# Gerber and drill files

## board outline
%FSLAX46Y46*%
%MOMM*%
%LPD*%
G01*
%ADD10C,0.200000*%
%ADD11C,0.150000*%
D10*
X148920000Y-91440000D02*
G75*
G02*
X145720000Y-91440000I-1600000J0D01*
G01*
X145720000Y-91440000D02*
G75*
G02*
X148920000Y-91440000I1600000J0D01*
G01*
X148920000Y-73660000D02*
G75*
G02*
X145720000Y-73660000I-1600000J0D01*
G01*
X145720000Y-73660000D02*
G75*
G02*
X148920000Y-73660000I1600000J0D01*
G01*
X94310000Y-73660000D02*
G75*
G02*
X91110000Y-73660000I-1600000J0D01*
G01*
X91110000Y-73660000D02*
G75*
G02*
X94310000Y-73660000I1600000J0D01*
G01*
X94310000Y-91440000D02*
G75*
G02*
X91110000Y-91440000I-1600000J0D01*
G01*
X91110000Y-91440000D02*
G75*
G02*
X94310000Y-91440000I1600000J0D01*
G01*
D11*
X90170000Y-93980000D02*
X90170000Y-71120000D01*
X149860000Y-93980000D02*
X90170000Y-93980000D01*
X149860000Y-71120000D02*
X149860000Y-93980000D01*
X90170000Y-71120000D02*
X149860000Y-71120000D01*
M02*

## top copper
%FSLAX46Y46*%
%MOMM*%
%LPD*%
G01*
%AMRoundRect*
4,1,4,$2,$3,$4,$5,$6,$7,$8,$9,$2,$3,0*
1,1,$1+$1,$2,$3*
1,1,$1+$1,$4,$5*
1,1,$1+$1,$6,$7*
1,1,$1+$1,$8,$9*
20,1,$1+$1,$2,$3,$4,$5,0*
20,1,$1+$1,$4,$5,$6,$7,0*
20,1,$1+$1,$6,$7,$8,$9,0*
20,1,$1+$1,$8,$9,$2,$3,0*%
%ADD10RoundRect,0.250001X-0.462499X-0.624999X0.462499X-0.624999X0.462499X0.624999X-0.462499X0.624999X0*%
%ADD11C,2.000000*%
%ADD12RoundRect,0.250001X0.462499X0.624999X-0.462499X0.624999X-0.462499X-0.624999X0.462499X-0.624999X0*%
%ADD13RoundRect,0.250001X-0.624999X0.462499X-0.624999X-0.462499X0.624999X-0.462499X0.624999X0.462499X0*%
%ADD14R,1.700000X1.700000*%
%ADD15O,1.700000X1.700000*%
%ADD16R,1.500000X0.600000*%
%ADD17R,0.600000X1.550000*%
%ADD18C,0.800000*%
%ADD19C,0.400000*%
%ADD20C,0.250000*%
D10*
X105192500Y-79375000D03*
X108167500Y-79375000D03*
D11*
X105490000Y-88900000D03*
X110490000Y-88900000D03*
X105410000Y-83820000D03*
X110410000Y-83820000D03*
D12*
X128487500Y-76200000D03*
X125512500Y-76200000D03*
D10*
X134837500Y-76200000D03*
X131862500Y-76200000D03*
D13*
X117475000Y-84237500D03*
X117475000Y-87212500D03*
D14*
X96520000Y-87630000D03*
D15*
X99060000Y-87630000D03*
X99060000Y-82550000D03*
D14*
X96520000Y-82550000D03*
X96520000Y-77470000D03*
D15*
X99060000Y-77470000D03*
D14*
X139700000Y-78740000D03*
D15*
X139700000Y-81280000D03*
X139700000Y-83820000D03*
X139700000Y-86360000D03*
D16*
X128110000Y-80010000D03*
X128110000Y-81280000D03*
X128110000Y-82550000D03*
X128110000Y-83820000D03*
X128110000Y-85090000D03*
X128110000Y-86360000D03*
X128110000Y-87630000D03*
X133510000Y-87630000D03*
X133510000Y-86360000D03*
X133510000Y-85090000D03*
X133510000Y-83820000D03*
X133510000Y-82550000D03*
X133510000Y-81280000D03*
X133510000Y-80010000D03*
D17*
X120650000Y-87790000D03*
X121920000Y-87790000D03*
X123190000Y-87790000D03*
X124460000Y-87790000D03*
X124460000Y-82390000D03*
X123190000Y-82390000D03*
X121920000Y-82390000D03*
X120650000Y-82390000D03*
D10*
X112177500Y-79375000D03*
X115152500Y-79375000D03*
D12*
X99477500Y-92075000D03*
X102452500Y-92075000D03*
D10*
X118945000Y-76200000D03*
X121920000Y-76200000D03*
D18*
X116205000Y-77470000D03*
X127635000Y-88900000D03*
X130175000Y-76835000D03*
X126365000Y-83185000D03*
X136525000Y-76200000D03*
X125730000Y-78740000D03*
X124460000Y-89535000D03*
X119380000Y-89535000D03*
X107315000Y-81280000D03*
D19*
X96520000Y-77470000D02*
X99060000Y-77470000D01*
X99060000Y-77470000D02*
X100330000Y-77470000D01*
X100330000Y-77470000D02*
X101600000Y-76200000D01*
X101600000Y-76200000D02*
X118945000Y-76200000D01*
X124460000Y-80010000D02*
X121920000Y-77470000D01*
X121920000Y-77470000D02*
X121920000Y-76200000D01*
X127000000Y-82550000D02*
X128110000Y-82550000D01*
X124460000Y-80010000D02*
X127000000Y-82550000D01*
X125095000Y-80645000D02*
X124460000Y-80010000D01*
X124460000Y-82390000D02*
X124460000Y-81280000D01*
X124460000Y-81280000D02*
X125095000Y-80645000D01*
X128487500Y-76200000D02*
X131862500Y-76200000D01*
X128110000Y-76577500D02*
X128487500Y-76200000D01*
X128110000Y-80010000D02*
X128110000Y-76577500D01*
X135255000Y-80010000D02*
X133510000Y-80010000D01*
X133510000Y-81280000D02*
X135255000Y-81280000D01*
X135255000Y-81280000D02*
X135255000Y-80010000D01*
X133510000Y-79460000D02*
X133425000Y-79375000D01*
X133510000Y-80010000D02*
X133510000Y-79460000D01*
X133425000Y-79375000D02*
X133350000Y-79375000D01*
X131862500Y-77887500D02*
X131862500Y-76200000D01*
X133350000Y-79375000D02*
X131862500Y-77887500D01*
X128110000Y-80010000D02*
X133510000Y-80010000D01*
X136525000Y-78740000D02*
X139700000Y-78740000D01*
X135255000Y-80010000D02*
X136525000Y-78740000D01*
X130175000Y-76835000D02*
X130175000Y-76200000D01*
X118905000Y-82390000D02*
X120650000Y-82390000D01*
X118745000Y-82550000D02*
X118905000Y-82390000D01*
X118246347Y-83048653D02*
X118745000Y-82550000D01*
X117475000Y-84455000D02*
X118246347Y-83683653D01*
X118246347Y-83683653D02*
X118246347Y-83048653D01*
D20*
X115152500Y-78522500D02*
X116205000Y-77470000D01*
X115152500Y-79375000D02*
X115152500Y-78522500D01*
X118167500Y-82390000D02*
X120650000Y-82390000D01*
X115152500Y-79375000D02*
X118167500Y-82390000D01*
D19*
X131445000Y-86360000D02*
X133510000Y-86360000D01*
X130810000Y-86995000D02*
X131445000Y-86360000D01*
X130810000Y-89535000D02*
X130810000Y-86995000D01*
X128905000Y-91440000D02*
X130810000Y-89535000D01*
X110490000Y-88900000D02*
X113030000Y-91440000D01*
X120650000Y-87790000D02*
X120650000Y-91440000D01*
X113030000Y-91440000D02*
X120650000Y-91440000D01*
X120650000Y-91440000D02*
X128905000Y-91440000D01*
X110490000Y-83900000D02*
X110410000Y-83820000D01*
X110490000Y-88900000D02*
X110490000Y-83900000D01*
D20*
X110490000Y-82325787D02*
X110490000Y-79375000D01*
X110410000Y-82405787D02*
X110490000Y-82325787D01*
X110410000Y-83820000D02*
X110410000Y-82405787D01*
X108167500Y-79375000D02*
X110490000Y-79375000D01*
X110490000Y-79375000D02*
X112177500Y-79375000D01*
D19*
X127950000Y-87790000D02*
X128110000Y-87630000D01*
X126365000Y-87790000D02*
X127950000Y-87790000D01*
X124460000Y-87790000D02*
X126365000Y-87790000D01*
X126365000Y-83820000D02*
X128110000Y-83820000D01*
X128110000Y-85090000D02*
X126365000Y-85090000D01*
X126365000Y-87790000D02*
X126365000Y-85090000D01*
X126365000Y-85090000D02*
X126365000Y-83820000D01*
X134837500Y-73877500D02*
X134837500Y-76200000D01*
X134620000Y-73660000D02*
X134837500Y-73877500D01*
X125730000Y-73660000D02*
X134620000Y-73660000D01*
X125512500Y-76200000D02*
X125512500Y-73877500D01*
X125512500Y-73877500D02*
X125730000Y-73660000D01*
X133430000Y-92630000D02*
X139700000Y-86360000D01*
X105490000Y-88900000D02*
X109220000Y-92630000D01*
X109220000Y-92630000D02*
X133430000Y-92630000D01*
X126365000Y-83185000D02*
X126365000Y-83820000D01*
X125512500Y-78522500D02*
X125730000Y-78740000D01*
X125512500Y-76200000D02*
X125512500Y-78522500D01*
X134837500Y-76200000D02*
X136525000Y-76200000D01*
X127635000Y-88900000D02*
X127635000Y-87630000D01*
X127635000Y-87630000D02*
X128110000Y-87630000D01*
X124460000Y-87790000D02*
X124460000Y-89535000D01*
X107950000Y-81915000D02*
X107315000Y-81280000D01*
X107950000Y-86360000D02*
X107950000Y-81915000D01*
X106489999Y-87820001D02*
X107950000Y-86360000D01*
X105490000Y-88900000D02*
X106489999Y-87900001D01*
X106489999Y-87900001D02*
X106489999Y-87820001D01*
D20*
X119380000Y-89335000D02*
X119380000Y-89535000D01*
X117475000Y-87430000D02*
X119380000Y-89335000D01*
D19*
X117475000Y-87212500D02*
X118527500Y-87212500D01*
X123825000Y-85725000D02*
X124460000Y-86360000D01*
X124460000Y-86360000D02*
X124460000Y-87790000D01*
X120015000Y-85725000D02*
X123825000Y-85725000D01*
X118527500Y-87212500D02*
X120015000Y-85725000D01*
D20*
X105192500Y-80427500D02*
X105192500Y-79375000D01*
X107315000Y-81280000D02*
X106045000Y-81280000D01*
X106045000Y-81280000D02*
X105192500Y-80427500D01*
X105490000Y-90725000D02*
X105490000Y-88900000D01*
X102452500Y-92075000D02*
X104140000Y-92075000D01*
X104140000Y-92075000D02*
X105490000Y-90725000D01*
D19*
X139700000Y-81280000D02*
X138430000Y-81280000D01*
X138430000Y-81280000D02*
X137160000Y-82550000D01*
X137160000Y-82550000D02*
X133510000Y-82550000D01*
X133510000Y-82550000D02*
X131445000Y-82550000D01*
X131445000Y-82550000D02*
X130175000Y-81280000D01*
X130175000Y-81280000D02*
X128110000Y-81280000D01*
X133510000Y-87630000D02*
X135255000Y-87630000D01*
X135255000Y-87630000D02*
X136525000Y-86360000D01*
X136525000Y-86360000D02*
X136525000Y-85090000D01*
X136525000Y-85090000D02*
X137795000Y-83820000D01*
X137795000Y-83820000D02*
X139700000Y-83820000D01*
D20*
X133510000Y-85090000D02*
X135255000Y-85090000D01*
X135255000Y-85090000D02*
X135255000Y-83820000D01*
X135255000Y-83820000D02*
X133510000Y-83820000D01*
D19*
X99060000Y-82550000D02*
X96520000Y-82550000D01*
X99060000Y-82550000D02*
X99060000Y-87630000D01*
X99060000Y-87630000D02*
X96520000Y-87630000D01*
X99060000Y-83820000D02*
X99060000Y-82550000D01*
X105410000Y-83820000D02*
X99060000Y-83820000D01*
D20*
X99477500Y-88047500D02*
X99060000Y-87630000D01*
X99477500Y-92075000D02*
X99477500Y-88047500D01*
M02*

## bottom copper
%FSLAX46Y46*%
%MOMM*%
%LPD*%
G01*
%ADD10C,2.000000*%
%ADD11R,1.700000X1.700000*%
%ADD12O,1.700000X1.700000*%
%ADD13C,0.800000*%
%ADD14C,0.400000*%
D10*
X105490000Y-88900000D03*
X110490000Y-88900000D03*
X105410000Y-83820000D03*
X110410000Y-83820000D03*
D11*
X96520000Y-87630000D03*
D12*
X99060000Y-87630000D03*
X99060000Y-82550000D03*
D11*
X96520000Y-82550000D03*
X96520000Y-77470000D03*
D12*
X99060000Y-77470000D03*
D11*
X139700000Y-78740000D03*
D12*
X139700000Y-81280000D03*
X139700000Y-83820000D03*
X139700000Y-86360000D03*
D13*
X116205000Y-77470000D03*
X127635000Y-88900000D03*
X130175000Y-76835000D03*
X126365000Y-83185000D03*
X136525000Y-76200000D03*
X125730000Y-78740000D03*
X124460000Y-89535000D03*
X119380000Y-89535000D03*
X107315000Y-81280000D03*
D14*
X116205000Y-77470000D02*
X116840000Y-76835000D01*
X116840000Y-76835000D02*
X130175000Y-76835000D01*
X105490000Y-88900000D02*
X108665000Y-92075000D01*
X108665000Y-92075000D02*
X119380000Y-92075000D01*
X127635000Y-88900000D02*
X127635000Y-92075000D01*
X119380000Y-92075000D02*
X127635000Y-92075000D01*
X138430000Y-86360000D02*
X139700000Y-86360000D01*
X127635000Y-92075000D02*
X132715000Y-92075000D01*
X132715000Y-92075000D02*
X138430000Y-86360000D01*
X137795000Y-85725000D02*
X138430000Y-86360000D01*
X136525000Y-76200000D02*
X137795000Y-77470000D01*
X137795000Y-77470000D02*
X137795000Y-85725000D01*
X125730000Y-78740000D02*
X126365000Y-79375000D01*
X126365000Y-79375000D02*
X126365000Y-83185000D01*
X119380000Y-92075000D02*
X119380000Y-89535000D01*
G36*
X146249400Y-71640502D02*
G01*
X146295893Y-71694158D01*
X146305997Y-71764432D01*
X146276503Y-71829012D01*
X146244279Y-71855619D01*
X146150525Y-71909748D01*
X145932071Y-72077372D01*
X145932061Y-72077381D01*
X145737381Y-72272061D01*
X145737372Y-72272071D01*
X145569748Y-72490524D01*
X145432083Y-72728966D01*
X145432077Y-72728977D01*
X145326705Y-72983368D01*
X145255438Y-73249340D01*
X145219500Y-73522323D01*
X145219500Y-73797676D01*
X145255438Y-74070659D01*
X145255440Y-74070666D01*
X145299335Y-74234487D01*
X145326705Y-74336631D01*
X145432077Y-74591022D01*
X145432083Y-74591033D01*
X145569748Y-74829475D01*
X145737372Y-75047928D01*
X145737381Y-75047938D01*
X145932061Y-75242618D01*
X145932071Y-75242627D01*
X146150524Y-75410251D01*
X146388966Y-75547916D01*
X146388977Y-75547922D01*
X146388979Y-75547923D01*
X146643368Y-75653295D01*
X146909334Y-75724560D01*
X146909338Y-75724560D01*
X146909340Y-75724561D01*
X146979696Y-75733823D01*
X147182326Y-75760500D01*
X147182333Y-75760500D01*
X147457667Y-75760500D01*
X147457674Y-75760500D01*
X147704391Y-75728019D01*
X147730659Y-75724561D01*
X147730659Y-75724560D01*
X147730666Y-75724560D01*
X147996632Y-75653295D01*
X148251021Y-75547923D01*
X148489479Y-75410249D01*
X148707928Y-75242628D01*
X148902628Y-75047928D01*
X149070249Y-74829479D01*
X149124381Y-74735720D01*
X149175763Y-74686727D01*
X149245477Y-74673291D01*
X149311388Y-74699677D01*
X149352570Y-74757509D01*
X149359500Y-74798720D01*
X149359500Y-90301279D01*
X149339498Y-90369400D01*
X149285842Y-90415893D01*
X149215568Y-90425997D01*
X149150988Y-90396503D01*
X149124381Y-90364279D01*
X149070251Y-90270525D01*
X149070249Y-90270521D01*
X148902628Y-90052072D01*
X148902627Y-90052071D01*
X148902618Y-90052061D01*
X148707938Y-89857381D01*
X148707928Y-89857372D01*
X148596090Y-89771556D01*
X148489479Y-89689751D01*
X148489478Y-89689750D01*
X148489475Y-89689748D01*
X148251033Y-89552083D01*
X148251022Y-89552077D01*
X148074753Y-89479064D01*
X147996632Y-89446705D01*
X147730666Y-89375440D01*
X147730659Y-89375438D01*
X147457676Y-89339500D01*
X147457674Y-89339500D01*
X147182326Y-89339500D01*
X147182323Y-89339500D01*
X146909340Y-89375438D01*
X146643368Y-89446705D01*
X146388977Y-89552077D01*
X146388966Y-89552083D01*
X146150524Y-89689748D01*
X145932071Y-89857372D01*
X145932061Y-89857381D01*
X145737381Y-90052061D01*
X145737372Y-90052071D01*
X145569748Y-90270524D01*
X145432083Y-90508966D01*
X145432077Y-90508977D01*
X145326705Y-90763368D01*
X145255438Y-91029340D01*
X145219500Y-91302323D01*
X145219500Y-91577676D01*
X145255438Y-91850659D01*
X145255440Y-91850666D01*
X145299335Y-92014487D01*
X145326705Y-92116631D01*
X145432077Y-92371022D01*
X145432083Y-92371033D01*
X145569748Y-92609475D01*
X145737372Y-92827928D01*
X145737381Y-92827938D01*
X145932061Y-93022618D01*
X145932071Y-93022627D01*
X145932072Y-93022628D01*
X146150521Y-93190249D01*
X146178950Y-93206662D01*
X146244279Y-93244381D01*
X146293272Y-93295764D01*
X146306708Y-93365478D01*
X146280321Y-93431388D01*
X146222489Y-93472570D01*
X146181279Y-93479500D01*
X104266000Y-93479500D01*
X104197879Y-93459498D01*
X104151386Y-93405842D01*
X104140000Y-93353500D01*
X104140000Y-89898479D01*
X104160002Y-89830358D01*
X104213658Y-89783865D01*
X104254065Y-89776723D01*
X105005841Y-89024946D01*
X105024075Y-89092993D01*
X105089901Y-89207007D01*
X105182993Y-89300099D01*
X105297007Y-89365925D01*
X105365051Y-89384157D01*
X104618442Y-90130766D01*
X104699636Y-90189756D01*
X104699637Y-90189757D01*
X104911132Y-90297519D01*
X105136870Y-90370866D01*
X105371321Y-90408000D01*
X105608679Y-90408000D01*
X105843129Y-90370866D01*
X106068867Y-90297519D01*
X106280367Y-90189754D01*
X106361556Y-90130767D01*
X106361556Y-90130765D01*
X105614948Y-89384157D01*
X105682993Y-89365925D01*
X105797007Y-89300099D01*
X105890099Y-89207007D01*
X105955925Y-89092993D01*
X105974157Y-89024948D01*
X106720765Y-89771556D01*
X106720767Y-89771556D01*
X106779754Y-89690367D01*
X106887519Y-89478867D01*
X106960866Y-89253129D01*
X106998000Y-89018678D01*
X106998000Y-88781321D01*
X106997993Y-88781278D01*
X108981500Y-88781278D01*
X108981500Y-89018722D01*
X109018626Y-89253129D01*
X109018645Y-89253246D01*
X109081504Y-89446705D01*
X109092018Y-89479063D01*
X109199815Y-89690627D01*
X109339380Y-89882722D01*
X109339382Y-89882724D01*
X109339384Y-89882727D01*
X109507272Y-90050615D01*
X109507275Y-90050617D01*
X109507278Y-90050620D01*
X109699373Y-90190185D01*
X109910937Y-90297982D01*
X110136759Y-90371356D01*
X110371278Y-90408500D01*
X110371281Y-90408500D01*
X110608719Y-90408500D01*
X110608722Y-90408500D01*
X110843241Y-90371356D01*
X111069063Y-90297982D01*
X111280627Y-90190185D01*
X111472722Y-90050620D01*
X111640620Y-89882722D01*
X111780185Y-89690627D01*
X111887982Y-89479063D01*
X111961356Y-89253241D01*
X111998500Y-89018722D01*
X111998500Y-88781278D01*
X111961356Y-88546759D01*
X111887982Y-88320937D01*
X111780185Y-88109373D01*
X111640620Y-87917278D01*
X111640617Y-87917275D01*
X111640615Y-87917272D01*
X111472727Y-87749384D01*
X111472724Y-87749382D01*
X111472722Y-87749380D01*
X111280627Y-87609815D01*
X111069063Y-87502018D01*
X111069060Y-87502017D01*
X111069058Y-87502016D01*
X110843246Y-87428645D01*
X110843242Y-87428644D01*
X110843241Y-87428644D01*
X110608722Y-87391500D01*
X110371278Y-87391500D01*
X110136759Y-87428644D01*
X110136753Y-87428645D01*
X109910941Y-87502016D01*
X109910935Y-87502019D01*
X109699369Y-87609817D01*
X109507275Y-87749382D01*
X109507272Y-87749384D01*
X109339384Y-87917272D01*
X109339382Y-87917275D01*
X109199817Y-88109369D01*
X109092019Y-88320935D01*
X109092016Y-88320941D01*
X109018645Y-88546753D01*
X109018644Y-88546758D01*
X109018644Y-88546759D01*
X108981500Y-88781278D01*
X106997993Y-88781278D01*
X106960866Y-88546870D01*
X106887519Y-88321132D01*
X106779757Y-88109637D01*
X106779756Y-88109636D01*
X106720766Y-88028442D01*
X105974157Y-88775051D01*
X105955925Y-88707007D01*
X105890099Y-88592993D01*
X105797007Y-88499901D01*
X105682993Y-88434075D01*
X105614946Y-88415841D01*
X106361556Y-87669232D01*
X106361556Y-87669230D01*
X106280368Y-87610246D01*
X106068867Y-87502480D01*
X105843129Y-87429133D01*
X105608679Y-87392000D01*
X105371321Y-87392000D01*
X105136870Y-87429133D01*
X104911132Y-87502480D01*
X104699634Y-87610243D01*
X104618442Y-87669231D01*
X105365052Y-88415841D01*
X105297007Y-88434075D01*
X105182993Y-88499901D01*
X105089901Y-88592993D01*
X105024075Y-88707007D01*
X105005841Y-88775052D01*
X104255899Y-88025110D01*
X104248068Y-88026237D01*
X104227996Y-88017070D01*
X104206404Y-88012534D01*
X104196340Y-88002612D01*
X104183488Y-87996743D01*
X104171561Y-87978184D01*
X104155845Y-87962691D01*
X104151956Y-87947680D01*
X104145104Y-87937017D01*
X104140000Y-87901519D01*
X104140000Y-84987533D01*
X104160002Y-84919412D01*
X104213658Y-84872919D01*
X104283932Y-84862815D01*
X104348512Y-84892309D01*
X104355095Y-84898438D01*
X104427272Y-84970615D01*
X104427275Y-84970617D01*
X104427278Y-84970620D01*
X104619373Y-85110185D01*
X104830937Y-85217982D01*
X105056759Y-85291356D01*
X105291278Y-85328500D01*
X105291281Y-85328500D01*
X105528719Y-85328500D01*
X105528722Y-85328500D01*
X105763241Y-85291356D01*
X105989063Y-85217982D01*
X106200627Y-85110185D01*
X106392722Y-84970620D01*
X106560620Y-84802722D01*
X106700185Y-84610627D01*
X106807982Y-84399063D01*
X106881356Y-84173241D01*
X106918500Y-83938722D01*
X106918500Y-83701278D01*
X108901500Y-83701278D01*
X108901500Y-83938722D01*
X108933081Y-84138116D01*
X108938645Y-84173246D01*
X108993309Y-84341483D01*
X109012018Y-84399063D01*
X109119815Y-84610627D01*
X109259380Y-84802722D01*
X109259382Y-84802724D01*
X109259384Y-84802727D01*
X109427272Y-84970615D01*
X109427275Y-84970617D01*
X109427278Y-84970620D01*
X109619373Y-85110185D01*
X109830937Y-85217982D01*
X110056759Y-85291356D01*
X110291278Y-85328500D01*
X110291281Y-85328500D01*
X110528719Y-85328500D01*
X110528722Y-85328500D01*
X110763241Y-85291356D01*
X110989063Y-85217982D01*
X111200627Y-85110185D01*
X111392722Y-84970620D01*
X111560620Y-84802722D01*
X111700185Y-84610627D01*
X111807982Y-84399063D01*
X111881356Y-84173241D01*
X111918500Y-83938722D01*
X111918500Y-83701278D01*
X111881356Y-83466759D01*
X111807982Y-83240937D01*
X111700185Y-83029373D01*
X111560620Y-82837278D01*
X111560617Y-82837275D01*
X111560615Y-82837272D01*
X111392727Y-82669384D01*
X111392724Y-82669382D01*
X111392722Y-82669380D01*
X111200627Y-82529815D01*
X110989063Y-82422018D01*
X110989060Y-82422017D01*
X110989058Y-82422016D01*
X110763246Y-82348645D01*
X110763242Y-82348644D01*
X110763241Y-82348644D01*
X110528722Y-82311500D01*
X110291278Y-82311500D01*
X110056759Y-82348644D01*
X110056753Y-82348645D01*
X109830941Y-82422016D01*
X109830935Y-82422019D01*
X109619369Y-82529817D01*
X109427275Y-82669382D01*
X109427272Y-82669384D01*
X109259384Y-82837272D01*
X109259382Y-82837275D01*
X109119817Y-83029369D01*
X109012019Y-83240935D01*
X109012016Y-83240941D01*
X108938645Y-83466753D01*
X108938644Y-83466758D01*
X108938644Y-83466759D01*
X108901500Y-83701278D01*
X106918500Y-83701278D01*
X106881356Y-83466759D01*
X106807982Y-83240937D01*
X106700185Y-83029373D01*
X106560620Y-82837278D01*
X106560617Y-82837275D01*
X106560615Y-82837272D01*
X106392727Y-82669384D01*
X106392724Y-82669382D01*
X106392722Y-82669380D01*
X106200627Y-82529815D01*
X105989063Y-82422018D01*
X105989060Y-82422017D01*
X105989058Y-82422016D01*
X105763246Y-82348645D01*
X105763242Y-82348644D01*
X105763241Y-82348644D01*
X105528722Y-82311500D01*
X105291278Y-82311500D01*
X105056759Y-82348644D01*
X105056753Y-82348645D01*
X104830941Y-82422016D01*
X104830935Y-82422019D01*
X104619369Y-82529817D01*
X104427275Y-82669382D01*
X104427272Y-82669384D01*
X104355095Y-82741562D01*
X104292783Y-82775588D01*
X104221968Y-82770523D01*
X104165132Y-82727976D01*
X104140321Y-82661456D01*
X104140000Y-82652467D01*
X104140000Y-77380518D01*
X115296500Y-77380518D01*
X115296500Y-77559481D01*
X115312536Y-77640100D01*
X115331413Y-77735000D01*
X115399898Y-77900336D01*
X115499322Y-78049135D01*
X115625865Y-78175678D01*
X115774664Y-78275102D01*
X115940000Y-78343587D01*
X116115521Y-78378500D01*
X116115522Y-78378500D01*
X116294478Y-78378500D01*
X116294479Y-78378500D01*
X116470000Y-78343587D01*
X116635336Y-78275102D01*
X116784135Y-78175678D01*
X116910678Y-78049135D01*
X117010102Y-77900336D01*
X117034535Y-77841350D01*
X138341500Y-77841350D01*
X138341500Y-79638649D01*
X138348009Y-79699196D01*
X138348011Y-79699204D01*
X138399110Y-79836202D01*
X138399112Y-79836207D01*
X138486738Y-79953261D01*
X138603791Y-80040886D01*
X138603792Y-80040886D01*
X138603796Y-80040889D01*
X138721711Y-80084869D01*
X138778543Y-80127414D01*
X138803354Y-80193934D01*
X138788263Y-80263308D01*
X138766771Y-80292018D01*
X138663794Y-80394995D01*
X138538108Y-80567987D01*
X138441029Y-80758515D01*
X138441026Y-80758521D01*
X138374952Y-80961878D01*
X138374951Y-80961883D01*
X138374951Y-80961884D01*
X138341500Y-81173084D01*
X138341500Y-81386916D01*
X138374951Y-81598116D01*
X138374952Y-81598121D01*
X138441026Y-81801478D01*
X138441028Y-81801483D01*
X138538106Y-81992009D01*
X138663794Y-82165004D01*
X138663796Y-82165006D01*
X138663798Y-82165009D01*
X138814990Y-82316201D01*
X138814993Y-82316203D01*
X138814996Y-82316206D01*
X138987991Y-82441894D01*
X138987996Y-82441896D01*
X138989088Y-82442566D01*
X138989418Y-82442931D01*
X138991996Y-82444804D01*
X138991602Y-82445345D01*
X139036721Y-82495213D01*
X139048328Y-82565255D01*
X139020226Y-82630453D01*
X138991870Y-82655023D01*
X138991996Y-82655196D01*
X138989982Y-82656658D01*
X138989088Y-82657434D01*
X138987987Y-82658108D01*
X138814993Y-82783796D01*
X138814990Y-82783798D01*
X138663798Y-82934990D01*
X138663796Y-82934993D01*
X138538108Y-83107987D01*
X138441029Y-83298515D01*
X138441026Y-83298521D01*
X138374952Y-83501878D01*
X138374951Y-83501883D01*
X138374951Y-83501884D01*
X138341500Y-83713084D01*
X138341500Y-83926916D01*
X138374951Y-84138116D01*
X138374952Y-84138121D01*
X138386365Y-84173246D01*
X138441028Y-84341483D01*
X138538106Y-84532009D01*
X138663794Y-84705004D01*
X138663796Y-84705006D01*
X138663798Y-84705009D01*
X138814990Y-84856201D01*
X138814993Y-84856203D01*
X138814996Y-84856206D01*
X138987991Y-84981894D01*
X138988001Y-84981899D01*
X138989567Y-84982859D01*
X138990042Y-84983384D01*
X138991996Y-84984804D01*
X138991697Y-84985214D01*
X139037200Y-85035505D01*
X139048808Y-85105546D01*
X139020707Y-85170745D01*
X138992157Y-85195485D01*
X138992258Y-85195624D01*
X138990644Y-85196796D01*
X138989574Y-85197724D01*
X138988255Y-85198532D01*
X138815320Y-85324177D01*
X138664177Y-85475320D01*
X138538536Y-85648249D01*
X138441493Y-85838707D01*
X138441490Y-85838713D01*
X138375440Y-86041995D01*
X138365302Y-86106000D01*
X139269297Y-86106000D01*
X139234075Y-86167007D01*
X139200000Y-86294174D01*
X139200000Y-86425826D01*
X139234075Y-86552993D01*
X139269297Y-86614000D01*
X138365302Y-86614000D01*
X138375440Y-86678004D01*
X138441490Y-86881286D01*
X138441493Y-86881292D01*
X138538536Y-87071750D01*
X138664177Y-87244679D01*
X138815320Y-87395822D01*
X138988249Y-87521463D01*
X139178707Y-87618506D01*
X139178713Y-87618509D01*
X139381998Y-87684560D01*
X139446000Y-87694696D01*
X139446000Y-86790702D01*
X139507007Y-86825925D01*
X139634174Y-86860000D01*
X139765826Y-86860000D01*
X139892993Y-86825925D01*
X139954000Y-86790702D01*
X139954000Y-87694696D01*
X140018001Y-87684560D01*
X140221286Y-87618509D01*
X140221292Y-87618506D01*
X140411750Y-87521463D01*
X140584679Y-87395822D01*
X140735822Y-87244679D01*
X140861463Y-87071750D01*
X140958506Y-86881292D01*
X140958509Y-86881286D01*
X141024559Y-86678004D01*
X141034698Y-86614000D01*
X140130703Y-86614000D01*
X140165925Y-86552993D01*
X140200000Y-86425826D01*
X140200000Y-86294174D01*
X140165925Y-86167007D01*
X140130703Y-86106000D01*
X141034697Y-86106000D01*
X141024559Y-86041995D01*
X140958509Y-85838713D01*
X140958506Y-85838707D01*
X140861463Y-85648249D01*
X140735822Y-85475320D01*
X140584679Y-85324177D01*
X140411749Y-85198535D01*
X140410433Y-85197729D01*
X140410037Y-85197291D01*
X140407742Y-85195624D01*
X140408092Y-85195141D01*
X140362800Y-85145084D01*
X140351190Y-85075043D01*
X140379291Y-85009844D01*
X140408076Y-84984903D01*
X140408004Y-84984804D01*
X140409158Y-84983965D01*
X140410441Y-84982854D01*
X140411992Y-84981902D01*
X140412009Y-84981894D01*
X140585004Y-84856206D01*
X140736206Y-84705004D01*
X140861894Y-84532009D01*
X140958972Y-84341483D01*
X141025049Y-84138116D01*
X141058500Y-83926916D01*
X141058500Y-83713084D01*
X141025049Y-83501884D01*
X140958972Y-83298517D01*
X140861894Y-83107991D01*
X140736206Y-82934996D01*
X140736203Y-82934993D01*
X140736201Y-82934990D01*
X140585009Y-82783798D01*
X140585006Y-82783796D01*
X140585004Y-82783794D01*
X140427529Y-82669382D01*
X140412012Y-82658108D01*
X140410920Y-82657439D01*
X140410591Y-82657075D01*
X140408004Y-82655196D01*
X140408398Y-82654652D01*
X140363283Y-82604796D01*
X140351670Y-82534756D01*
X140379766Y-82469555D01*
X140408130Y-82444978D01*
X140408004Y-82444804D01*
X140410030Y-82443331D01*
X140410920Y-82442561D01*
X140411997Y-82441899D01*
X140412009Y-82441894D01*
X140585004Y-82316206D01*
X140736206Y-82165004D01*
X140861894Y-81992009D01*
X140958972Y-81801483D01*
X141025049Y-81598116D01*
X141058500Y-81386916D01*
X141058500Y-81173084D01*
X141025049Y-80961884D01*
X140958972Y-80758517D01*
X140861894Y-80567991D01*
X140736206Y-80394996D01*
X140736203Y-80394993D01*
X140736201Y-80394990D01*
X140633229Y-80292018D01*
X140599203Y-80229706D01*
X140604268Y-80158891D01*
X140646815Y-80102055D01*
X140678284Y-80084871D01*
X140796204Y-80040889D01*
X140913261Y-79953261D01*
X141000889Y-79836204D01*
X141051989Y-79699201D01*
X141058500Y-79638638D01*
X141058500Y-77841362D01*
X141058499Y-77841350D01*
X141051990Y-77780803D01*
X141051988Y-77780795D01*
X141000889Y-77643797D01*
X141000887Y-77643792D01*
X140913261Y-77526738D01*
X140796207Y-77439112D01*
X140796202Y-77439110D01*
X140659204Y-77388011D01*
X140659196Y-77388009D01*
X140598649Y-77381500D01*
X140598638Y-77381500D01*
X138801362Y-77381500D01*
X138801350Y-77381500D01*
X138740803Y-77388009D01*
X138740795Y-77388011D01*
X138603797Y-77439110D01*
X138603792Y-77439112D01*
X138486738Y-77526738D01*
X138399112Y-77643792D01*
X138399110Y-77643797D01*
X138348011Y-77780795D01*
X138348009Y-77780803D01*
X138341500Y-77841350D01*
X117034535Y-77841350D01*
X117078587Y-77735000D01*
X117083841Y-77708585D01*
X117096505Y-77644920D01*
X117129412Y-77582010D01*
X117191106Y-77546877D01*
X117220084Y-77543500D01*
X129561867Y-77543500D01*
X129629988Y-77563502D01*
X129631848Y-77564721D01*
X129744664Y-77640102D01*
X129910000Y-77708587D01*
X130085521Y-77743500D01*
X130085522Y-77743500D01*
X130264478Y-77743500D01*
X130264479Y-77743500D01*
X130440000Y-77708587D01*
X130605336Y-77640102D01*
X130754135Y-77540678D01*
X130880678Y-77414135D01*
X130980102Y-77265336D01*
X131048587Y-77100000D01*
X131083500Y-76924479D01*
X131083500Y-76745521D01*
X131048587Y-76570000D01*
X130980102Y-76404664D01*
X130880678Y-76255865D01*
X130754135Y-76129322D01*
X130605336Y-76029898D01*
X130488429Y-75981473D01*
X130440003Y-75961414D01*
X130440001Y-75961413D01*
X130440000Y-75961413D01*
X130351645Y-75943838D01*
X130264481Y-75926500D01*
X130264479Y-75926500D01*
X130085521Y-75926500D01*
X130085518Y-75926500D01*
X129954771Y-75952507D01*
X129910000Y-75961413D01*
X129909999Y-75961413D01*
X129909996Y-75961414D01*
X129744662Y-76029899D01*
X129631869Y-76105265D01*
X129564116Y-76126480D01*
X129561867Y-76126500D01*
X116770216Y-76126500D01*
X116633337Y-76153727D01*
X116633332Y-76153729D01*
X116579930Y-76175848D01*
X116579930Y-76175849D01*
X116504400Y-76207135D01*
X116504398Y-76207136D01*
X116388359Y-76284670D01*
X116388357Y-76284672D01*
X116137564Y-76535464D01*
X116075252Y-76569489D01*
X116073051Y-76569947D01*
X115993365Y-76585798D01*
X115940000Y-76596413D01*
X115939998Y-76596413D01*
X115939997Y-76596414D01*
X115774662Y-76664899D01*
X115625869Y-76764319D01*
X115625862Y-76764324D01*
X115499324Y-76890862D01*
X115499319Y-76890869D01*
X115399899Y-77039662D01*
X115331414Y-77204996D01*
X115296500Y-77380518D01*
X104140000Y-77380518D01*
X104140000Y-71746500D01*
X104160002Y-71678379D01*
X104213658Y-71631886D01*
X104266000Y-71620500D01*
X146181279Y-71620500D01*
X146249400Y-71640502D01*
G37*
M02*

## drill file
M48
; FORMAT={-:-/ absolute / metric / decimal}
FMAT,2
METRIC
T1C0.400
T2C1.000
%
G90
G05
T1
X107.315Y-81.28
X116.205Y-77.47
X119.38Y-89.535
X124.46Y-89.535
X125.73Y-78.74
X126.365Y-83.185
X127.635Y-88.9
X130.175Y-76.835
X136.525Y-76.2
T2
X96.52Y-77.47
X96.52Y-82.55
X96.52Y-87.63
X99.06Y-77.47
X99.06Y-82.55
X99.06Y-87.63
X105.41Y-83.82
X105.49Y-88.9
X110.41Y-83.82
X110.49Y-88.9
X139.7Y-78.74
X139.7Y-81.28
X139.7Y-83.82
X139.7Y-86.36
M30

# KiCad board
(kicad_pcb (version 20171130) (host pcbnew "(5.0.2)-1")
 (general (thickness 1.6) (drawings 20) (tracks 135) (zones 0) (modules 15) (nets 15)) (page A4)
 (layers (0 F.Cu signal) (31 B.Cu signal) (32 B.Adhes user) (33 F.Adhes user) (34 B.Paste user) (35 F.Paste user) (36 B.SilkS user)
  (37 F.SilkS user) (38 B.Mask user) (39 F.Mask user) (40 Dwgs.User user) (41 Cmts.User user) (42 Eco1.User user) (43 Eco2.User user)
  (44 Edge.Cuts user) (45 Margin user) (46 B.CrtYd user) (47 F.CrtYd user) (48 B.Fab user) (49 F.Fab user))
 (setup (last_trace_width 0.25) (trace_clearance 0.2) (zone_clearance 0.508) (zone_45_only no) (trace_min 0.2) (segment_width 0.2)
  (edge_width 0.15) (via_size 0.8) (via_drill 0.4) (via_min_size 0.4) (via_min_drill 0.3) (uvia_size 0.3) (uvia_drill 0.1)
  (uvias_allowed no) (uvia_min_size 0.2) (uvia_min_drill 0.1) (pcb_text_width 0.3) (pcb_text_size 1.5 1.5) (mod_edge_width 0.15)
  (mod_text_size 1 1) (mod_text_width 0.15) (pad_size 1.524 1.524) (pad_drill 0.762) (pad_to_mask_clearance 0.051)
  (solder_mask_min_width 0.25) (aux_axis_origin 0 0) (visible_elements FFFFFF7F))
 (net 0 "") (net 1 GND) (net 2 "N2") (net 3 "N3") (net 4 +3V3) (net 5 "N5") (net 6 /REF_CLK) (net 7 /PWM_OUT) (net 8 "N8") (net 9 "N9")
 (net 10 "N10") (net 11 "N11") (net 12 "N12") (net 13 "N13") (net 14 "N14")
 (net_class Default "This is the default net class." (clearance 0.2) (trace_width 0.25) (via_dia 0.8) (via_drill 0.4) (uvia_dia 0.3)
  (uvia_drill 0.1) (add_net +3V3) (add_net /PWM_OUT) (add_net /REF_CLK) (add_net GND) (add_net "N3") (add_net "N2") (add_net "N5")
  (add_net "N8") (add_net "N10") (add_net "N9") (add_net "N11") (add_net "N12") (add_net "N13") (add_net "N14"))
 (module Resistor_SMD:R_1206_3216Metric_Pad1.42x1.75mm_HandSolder (layer F.Cu) (at 106.68 79.375)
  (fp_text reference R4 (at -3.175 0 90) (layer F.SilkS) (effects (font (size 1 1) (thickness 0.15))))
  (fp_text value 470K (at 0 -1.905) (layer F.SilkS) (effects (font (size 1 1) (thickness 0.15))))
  (pad 1 smd roundrect (at -1.4875 0) (size 1.425 1.75) (layers F.Cu F.Paste F.Mask) (roundrect_rratio 0.175439) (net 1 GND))
  (pad 2 smd roundrect (at 1.4875 0) (size 1.425 1.75) (layers F.Cu F.Paste F.Mask) (roundrect_rratio 0.175439) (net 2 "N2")))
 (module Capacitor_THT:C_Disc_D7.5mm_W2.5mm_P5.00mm (layer F.Cu) (at 110.49 88.9 180)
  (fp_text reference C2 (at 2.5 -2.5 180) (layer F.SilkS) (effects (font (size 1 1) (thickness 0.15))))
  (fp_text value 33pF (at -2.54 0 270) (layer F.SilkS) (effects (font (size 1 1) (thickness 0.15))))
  (pad 2 thru_hole circle (at 5 0 180) (size 2 2) (drill 1) (layers *.Cu *.Mask) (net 1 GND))
  (pad 1 thru_hole circle (at 0 0 180) (size 2 2) (drill 1) (layers *.Cu *.Mask) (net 2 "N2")))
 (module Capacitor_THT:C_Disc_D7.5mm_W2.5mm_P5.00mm (layer F.Cu) (at 105.41 83.82)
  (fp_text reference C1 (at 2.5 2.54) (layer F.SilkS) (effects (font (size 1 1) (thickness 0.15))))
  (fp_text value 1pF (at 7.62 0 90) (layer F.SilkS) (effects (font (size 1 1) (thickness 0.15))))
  (pad 1 thru_hole circle (at 0 0) (size 2 2) (drill 1) (layers *.Cu *.Mask) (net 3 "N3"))
  (pad 2 thru_hole circle (at 5 0) (size 2 2) (drill 1) (layers *.Cu *.Mask) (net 2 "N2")))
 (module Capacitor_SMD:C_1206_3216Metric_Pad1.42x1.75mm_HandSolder (layer F.Cu) (at 127 76.2 180)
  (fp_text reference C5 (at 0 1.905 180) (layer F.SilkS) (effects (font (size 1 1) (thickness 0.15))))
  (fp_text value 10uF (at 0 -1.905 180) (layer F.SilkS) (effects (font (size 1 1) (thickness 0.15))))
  (pad 1 smd roundrect (at -1.4875 0 180) (size 1.425 1.75) (layers F.Cu F.Paste F.Mask) (roundrect_rratio 0.175439) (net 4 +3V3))
  (pad 2 smd roundrect (at 1.4875 0 180) (size 1.425 1.75) (layers F.Cu F.Paste F.Mask) (roundrect_rratio 0.175439) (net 1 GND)))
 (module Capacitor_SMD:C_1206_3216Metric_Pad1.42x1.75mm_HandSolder (layer F.Cu) (at 133.35 76.2)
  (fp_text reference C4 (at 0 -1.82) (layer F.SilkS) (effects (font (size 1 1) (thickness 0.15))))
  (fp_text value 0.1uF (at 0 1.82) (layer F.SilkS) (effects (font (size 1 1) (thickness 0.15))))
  (pad 2 smd roundrect (at 1.4875 0) (size 1.425 1.75) (layers F.Cu F.Paste F.Mask) (roundrect_rratio 0.175439) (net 1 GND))
  (pad 1 smd roundrect (at -1.4875 0) (size 1.425 1.75) (layers F.Cu F.Paste F.Mask) (roundrect_rratio 0.175439) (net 4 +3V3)))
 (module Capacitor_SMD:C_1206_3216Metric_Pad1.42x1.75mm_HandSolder (layer F.Cu) (at 117.475 85.725 270)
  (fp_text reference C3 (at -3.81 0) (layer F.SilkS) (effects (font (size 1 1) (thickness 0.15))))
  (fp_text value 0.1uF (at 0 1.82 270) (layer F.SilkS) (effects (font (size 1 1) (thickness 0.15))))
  (pad 1 smd roundrect (at -1.4875 0 270) (size 1.425 1.75) (layers F.Cu F.Paste F.Mask) (roundrect_rratio 0.175439) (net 4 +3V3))
  (pad 2 smd roundrect (at 1.4875 0 270) (size 1.425 1.75) (layers F.Cu F.Paste F.Mask) (roundrect_rratio 0.175439) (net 1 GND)))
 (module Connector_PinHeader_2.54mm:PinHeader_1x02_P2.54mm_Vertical (layer F.Cu) (at 96.52 87.63 90)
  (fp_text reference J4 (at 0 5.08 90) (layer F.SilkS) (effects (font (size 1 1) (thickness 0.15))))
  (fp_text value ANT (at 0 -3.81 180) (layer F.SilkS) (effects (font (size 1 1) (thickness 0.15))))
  (pad 1 thru_hole rect (at 0 0 90) (size 1.7 1.7) (drill 1) (layers *.Cu *.Mask) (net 3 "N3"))
  (pad 2 thru_hole oval (at 0 2.54 90) (size 1.7 1.7) (drill 1) (layers *.Cu *.Mask) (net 3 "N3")))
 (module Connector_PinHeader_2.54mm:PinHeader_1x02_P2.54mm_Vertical (layer F.Cu) (at 96.52 82.55 90)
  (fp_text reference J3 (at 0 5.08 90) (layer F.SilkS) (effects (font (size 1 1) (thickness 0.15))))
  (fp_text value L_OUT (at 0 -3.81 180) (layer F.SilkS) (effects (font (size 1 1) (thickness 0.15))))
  (pad 2 thru_hole oval (at 0 2.54 90) (size 1.7 1.7) (drill 1) (layers *.Cu *.Mask) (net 3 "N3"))
  (pad 1 thru_hole rect (at 0 0 90) (size 1.7 1.7) (drill 1) (layers *.Cu *.Mask) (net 3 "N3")))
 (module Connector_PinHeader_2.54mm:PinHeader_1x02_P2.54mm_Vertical (layer F.Cu) (at 96.52 77.47 90)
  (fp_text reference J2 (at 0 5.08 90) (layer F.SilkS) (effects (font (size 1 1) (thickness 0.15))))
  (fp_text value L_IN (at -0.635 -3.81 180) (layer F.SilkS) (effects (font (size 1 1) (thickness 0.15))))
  (pad 1 thru_hole rect (at 0 0 90) (size 1.7 1.7) (drill 1) (layers *.Cu *.Mask) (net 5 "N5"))
  (pad 2 thru_hole oval (at 0 2.54 90) (size 1.7 1.7) (drill 1) (layers *.Cu *.Mask) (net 5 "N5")))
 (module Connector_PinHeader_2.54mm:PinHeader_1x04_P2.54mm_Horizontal (layer F.Cu) (at 139.7 78.74)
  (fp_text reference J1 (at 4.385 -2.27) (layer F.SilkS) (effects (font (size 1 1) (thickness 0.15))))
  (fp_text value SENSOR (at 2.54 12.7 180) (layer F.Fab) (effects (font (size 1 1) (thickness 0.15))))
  (pad 1 thru_hole rect (at 0 0) (size 1.7 1.7) (drill 1) (layers *.Cu *.Mask) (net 4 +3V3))
  (pad 2 thru_hole oval (at 0 2.54) (size 1.7 1.7) (drill 1) (layers *.Cu *.Mask) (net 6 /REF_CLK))
  (pad 3 thru_hole oval (at 0 5.08) (size 1.7 1.7) (drill 1) (layers *.Cu *.Mask) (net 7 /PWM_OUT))
  (pad 4 thru_hole oval (at 0 7.62) (size 1.7 1.7) (drill 1) (layers *.Cu *.Mask) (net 1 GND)))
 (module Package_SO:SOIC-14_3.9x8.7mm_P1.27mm (layer F.Cu) (at 130.81 83.82)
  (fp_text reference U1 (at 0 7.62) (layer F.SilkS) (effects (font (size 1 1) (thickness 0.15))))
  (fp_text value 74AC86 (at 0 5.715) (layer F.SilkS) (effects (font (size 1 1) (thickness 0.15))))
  (pad 1 smd rect (at -2.7 -3.81) (size 1.5 0.6) (layers F.Cu F.Paste F.Mask) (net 4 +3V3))
  (pad 2 smd rect (at -2.7 -2.54) (size 1.5 0.6) (layers F.Cu F.Paste F.Mask) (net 6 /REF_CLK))
  (pad 3 smd rect (at -2.7 -1.27) (size 1.5 0.6) (layers F.Cu F.Paste F.Mask) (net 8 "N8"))
  (pad 4 smd rect (at -2.7 0) (size 1.5 0.6) (layers F.Cu F.Paste F.Mask) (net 1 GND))
  (pad 5 smd rect (at -2.7 1.27) (size 1.5 0.6) (layers F.Cu F.Paste F.Mask) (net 1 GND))
  (pad 6 smd rect (at -2.7 2.54) (size 1.5 0.6) (layers F.Cu F.Paste F.Mask) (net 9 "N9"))
  (pad 7 smd rect (at -2.7 3.81) (size 1.5 0.6) (layers F.Cu F.Paste F.Mask) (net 1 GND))
  (pad 8 smd rect (at 2.7 3.81) (size 1.5 0.6) (layers F.Cu F.Paste F.Mask) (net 7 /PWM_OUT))
  (pad 9 smd rect (at 2.7 2.54) (size 1.5 0.6) (layers F.Cu F.Paste F.Mask) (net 2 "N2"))
  (pad 10 smd rect (at 2.7 1.27) (size 1.5 0.6) (layers F.Cu F.Paste F.Mask) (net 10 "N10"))
  (pad 11 smd rect (at 2.7 0) (size 1.5 0.6) (layers F.Cu F.Paste F.Mask) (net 10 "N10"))
  (pad 12 smd rect (at 2.7 -1.27) (size 1.5 0.6) (layers F.Cu F.Paste F.Mask) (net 6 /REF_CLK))
  (pad 13 smd rect (at 2.7 -2.54) (size 1.5 0.6) (layers F.Cu F.Paste F.Mask) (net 4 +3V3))
  (pad 14 smd rect (at 2.7 -3.81) (size 1.5 0.6) (layers F.Cu F.Paste F.Mask) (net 4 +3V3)))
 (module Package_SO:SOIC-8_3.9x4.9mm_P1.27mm (layer F.Cu) (at 122.555 85.09 90)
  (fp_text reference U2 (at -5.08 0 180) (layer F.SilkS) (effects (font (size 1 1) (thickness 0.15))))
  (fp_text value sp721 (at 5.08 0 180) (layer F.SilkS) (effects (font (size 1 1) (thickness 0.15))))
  (pad 1 smd rect (at -2.7 -1.905 90) (size 1.55 0.6) (layers F.Cu F.Paste F.Mask) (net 2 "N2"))
  (pad 2 smd rect (at -2.7 -0.635 90) (size 1.55 0.6) (layers F.Cu F.Paste F.Mask) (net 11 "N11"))
  (pad 3 smd rect (at -2.7 0.635 90) (size 1.55 0.6) (layers F.Cu F.Paste F.Mask) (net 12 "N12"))
  (pad 4 smd rect (at -2.7 1.905 90) (size 1.55 0.6) (layers F.Cu F.Paste F.Mask) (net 1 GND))
  (pad 5 smd rect (at 2.7 1.905 90) (size 1.55 0.6) (layers F.Cu F.Paste F.Mask) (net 8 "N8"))
  (pad 6 smd rect (at 2.7 0.635 90) (size 1.55 0.6) (layers F.Cu F.Paste F.Mask) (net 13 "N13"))
  (pad 7 smd rect (at 2.7 -0.635 90) (size 1.55 0.6) (layers F.Cu F.Paste F.Mask) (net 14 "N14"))
  (pad 8 smd rect (at 2.7 -1.905 90) (size 1.55 0.6) (layers F.Cu F.Paste F.Mask) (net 4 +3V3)))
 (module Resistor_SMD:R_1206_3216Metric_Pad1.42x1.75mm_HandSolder (layer F.Cu) (at 113.665 79.375)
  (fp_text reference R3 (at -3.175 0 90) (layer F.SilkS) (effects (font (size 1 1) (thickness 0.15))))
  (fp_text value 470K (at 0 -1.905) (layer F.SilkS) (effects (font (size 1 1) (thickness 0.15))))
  (pad 1 smd roundrect (at -1.4875 0) (size 1.425 1.75) (layers F.Cu F.Paste F.Mask) (roundrect_rratio 0.175439) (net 2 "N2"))
  (pad 2 smd roundrect (at 1.4875 0) (size 1.425 1.75) (layers F.Cu F.Paste F.Mask) (roundrect_rratio 0.175439) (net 4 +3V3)))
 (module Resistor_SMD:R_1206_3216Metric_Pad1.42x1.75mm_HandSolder (layer F.Cu) (at 100.965 92.075 180)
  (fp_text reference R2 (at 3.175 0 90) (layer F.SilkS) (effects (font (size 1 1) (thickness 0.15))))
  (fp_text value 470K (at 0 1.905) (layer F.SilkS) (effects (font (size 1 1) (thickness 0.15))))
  (pad 2 smd roundrect (at 1.4875 0 180) (size 1.425 1.75) (layers F.Cu F.Paste F.Mask) (roundrect_rratio 0.175439) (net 3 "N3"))
  (pad 1 smd roundrect (at -1.4875 0 180) (size 1.425 1.75) (layers F.Cu F.Paste F.Mask) (roundrect_rratio 0.175439) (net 1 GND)))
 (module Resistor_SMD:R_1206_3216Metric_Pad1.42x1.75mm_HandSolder (layer F.Cu) (at 120.4325 76.2)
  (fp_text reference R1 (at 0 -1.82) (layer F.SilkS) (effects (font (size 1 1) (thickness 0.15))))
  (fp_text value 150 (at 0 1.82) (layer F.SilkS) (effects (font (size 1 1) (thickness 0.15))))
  (pad 1 smd roundrect (at -1.4875 0) (size 1.425 1.75) (layers F.Cu F.Paste F.Mask) (roundrect_rratio 0.175439) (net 5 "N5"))
  (pad 2 smd roundrect (at 1.4875 0) (size 1.425 1.75) (layers F.Cu F.Paste F.Mask) (roundrect_rratio 0.175439) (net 8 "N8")))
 (gr_circle (center 147.32 91.44) (end 148.92 91.44) (layer Edge.Cuts) (width 0.2))
 (gr_circle (center 147.32 73.66) (end 148.92 73.66) (layer Edge.Cuts) (width 0.2))
 (gr_circle (center 92.71 73.66) (end 94.31 73.66) (layer Edge.Cuts) (width 0.2))
 (gr_circle (center 92.71 91.44) (end 94.31 91.44) (layer Edge.Cuts) (width 0.2))
 (gr_line (start 90.17 93.98) (end 90.17 71.12) (layer Edge.Cuts) (width 0.15))
 (gr_line (start 149.86 93.98) (end 90.17 93.98) (layer Edge.Cuts) (width 0.15))
 (gr_line (start 149.86 71.12) (end 149.86 93.98) (layer Edge.Cuts) (width 0.15))
 (gr_line (start 90.17 71.12) (end 149.86 71.12) (layer Edge.Cuts) (width 0.15))
 (via (at 116.205 77.47) (size 0.8) (drill 0.4) (layers F.Cu B.Cu) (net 4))
 (via (at 127.635 88.9) (size 0.8) (drill 0.4) (layers F.Cu B.Cu) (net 1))
 (segment (start 96.52 77.47) (end 99.06 77.47) (width 0.4) (layer F.Cu) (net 5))
 (segment (start 99.06 77.47) (end 100.33 77.47) (width 0.4) (layer F.Cu) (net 5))
 (segment (start 100.33 77.47) (end 101.6 76.2) (width 0.4) (layer F.Cu) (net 5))
 (segment (start 101.6 76.2) (end 118.945 76.2) (width 0.4) (layer F.Cu) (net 5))
 (segment (start 124.46 80.01) (end 121.92 77.47) (width 0.4) (layer F.Cu) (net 8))
 (segment (start 121.92 77.47) (end 121.92 76.2) (width 0.4) (layer F.Cu) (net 8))
 (segment (start 127 82.55) (end 128.11 82.55) (width 0.4) (layer F.Cu) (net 8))
 (segment (start 124.46 80.01) (end 127 82.55) (width 0.4) (layer F.Cu) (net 8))
 (segment (start 125.095 80.645) (end 124.46 80.01) (width 0.4) (layer F.Cu) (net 8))
 (segment (start 124.46 82.39) (end 124.46 81.28) (width 0.4) (layer F.Cu) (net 8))
 (segment (start 124.46 81.28) (end 125.095 80.645) (width 0.4) (layer F.Cu) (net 8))
 (segment (start 128.4875 76.2) (end 131.8625 76.2) (width 0.4) (layer F.Cu) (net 4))
 (segment (start 128.11 76.5775) (end 128.4875 76.2) (width 0.4) (layer F.Cu) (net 4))
 (segment (start 128.11 80.01) (end 128.11 76.5775) (width 0.4) (layer F.Cu) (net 4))
 (segment (start 135.255 80.01) (end 133.51 80.01) (width 0.4) (layer F.Cu) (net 4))
 (segment (start 133.51 81.28) (end 135.255 81.28) (width 0.4) (layer F.Cu) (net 4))
 (segment (start 135.255 81.28) (end 135.255 80.01) (width 0.4) (layer F.Cu) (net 4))
 (segment (start 133.51 79.46) (end 133.425 79.375) (width 0.4) (layer F.Cu) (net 4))
 (segment (start 133.51 80.01) (end 133.51 79.46) (width 0.4) (layer F.Cu) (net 4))
 (segment (start 133.425 79.375) (end 133.35 79.375) (width 0.4) (layer F.Cu) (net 4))
 (segment (start 131.8625 77.8875) (end 131.8625 76.2) (width 0.4) (layer F.Cu) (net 4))
 (segment (start 133.35 79.375) (end 131.8625 77.8875) (width 0.4) (layer F.Cu) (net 4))
 (segment (start 128.11 80.01) (end 133.51 80.01) (width 0.4) (layer F.Cu) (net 4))
 (segment (start 136.525 78.74) (end 139.7 78.74) (width 0.4) (layer F.Cu) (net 4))
 (segment (start 135.255 80.01) (end 136.525 78.74) (width 0.4) (layer F.Cu) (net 4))
 (via (at 130.175 76.835) (size 0.8) (drill 0.4) (layers F.Cu B.Cu) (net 4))
 (segment (start 130.175 76.835) (end 130.175 76.2) (width 0.4) (layer F.Cu) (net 4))
 (segment (start 116.205 77.47) (end 116.84 76.835) (width 0.4) (layer B.Cu) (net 4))
 (segment (start 116.84 76.835) (end 130.175 76.835) (width 0.4) (layer B.Cu) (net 4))
 (segment (start 118.905 82.39) (end 120.65 82.39) (width 0.4) (layer F.Cu) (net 4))
 (segment (start 118.745 82.55) (end 118.905 82.39) (width 0.4) (layer F.Cu) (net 4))
 (segment (start 118.246347 83.048653) (end 118.745 82.55) (width 0.4) (layer F.Cu) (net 4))
 (segment (start 117.475 84.455) (end 118.246347 83.683653) (width 0.4) (layer F.Cu) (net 4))
 (segment (start 118.246347 83.683653) (end 118.246347 83.048653) (width 0.4) (layer F.Cu) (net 4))
 (segment (start 115.1525 78.5225) (end 116.205 77.47) (width 0.25) (layer F.Cu) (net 4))
 (segment (start 115.1525 79.375) (end 115.1525 78.5225) (width 0.25) (layer F.Cu) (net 4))
 (segment (start 118.1675 82.39) (end 120.65 82.39) (width 0.25) (layer F.Cu) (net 4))
 (segment (start 115.1525 79.375) (end 118.1675 82.39) (width 0.25) (layer F.Cu) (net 4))
 (segment (start 131.445 86.36) (end 133.51 86.36) (width 0.4) (layer F.Cu) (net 2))
 (segment (start 130.81 86.995) (end 131.445 86.36) (width 0.4) (layer F.Cu) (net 2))
 (segment (start 130.81 89.535) (end 130.81 86.995) (width 0.4) (layer F.Cu) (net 2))
 (segment (start 128.905 91.44) (end 130.81 89.535) (width 0.4) (layer F.Cu) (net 2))
 (segment (start 110.49 88.9) (end 113.03 91.44) (width 0.4) (layer F.Cu) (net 2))
 (segment (start 120.65 87.79) (end 120.65 91.44) (width 0.4) (layer F.Cu) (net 2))
 (segment (start 113.03 91.44) (end 120.65 91.44) (width 0.4) (layer F.Cu) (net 2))
 (segment (start 120.65 91.44) (end 128.905 91.44) (width 0.4) (layer F.Cu) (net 2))
 (segment (start 110.49 83.9) (end 110.41 83.82) (width 0.4) (layer F.Cu) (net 2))
 (segment (start 110.49 88.9) (end 110.49 83.9) (width 0.4) (layer F.Cu) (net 2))
 (segment (start 110.49 82.325787) (end 110.49 79.375) (width 0.25) (layer F.Cu) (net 2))
 (segment (start 110.41 82.405787) (end 110.49 82.325787) (width 0.25) (layer F.Cu) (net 2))
 (segment (start 110.41 83.82) (end 110.41 82.405787) (width 0.25) (layer F.Cu) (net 2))
 (segment (start 108.1675 79.375) (end 110.49 79.375) (width 0.25) (layer F.Cu) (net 2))
 (segment (start 110.49 79.375) (end 112.1775 79.375) (width 0.25) (layer F.Cu) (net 2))
 (segment (start 127.95 87.79) (end 128.11 87.63) (width 0.4) (layer F.Cu) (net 1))
 (segment (start 126.365 87.79) (end 127.95 87.79) (width 0.4) (layer F.Cu) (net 1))
 (segment (start 124.46 87.79) (end 126.365 87.79) (width 0.4) (layer F.Cu) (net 1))
 (segment (start 126.365 83.82) (end 128.11 83.82) (width 0.4) (layer F.Cu) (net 1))
 (segment (start 128.11 85.09) (end 126.365 85.09) (width 0.4) (layer F.Cu) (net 1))
 (segment (start 126.365 87.79) (end 126.365 85.09) (width 0.4) (layer F.Cu) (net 1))
 (segment (start 126.365 85.09) (end 126.365 83.82) (width 0.4) (layer F.Cu) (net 1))
 (segment (start 134.8375 73.8775) (end 134.8375 76.2) (width 0.4) (layer F.Cu) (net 1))
 (segment (start 134.62 73.66) (end 134.8375 73.8775) (width 0.4) (layer F.Cu) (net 1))
 (segment (start 125.73 73.66) (end 134.62 73.66) (width 0.4) (layer F.Cu) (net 1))
 (segment (start 125.5125 76.2) (end 125.5125 73.8775) (width 0.4) (layer F.Cu) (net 1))
 (segment (start 125.5125 73.8775) (end 125.73 73.66) (width 0.4) (layer F.Cu) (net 1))
 (segment (start 133.43 92.63) (end 139.7 86.36) (width 0.4) (layer F.Cu) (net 1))
 (segment (start 105.49 88.9) (end 109.22 92.63) (width 0.4) (layer F.Cu) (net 1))
 (segment (start 109.22 92.63) (end 133.43 92.63) (width 0.4) (layer F.Cu) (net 1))
 (via (at 126.365 83.185) (size 0.8) (drill 0.4) (layers F.Cu B.Cu) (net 1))
 (segment (start 126.365 83.185) (end 126.365 83.82) (width 0.4) (layer F.Cu) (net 1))
 (via (at 136.525 76.2) (size 0.8) (drill 0.4) (layers F.Cu B.Cu) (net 1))
 (via (at 125.73 78.74) (size 0.8) (drill 0.4) (layers F.Cu B.Cu) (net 1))
 (segment (start 125.5125 78.5225) (end 125.73 78.74) (width 0.4) (layer F.Cu) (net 1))
 (segment (start 125.5125 76.2) (end 125.5125 78.5225) (width 0.4) (layer F.Cu) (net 1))
 (segment (start 134.8375 76.2) (end 136.525 76.2) (width 0.4) (layer F.Cu) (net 1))
 (segment (start 105.49 88.9) (end 108.665 92.075) (width 0.4) (layer B.Cu) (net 1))
 (segment (start 108.665 92.075) (end 119.38 92.075) (width 0.4) (layer B.Cu) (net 1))
 (segment (start 127.635 88.9) (end 127.635 92.075) (width 0.4) (layer B.Cu) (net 1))
 (segment (start 119.38 92.075) (end 127.635 92.075) (width 0.4) (layer B.Cu) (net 1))
 (segment (start 138.43 86.36) (end 139.7 86.36) (width 0.4) (layer B.Cu) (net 1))
 (segment (start 127.635 92.075) (end 132.715 92.075) (width 0.4) (layer B.Cu) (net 1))
 (segment (start 132.715 92.075) (end 138.43 86.36) (width 0.4) (layer B.Cu) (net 1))
 (segment (start 137.795 85.725) (end 138.43 86.36) (width 0.4) (layer B.Cu) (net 1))
 (segment (start 136.525 76.2) (end 137.795 77.47) (width 0.4) (layer B.Cu) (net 1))
 (segment (start 137.795 77.47) (end 137.795 85.725) (width 0.4) (layer B.Cu) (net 1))
 (segment (start 125.73 78.74) (end 126.365 79.375) (width 0.4) (layer B.Cu) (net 1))
 (segment (start 126.365 79.375) (end 126.365 83.185) (width 0.4) (layer B.Cu) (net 1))
 (segment (start 127.635 88.9) (end 127.635 87.63) (width 0.4) (layer F.Cu) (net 1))
 (segment (start 127.635 87.63) (end 128.11 87.63) (width 0.4) (layer F.Cu) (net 1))
 (via (at 124.46 89.535) (size 0.8) (drill 0.4) (layers F.Cu B.Cu) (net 1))
 (segment (start 124.46 87.79) (end 124.46 89.535) (width 0.4) (layer F.Cu) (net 1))
 (via (at 119.38 89.535) (size 0.8) (drill 0.4) (layers F.Cu B.Cu) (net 1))
 (segment (start 119.38 92.075) (end 119.38 89.535) (width 0.4) (layer B.Cu) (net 1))
 (via (at 107.315 81.28) (size 0.8) (drill 0.4) (layers F.Cu B.Cu) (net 1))
 (segment (start 107.95 81.915) (end 107.315 81.28) (width 0.4) (layer F.Cu) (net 1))
 (segment (start 107.95 86.36) (end 107.95 81.915) (width 0.4) (layer F.Cu) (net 1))
 (segment (start 106.489999 87.820001) (end 107.95 86.36) (width 0.4) (layer F.Cu) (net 1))
 (segment (start 105.49 88.9) (end 106.489999 87.900001) (width 0.4) (layer F.Cu) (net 1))
 (segment (start 106.489999 87.900001) (end 106.489999 87.820001) (width 0.4) (layer F.Cu) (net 1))
 (segment (start 119.38 89.335) (end 119.38 89.535) (width 0.25) (layer F.Cu) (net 1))
 (segment (start 117.475 87.43) (end 119.38 89.335) (width 0.25) (layer F.Cu) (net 1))
 (segment (start 117.475 87.2125) (end 118.5275 87.2125) (width 0.4) (layer F.Cu) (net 1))
 (segment (start 123.825 85.725) (end 124.46 86.36) (width 0.4) (layer F.Cu) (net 1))
 (segment (start 124.46 86.36) (end 124.46 87.79) (width 0.4) (layer F.Cu) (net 1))
 (segment (start 120.015 85.725) (end 123.825 85.725) (width 0.4) (layer F.Cu) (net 1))
 (segment (start 118.5275 87.2125) (end 120.015 85.725) (width 0.4) (layer F.Cu) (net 1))
 (segment (start 105.1925 80.4275) (end 105.1925 79.375) (width 0.25) (layer F.Cu) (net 1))
 (segment (start 107.315 81.28) (end 106.045 81.28) (width 0.25) (layer F.Cu) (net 1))
 (segment (start 106.045 81.28) (end 105.1925 80.4275) (width 0.25) (layer F.Cu) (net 1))
 (segment (start 105.49 90.725) (end 105.49 88.9) (width 0.25) (layer F.Cu) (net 1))
 (segment (start 102.4525 92.075) (end 104.14 92.075) (width 0.25) (layer F.Cu) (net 1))
 (segment (start 104.14 92.075) (end 105.49 90.725) (width 0.25) (layer F.Cu) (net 1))
 (segment (start 139.7 81.28) (end 138.43 81.28) (width 0.4) (layer F.Cu) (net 6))
 (segment (start 138.43 81.28) (end 137.16 82.55) (width 0.4) (layer F.Cu) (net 6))
 (segment (start 137.16 82.55) (end 133.51 82.55) (width 0.4) (layer F.Cu) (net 6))
 (segment (start 133.51 82.55) (end 131.445 82.55) (width 0.4) (layer F.Cu) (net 6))
 (segment (start 131.445 82.55) (end 130.175 81.28) (width 0.4) (layer F.Cu) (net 6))
 (segment (start 130.175 81.28) (end 128.11 81.28) (width 0.4) (layer F.Cu) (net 6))
 (segment (start 133.51 87.63) (end 135.255 87.63) (width 0.4) (layer F.Cu) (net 7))
 (segment (start 135.255 87.63) (end 136.525 86.36) (width 0.4) (layer F.Cu) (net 7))
 (segment (start 136.525 86.36) (end 136.525 85.09) (width 0.4) (layer F.Cu) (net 7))
 (segment (start 136.525 85.09) (end 137.795 83.82) (width 0.4) (layer F.Cu) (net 7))
 (segment (start 137.795 83.82) (end 139.7 83.82) (width 0.4) (layer F.Cu) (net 7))
 (segment (start 133.51 85.09) (end 135.255 85.09) (width 0.25) (layer F.Cu) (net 10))
 (segment (start 135.255 85.09) (end 135.255 83.82) (width 0.25) (layer F.Cu) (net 10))
 (segment (start 135.255 83.82) (end 133.51 83.82) (width 0.25) (layer F.Cu) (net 10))
 (segment (start 99.06 82.55) (end 96.52 82.55) (width 0.4) (layer F.Cu) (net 3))
 (segment (start 99.06 82.55) (end 99.06 87.63) (width 0.4) (layer F.Cu) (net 3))
 (segment (start 99.06 87.63) (end 96.52 87.63) (width 0.4) (layer F.Cu) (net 3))
 (segment (start 99.06 83.82) (end 99.06 82.55) (width 0.4) (layer F.Cu) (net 3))
 (segment (start 105.41 83.82) (end 99.06 83.82) (width 0.4) (layer F.Cu) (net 3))
 (segment (start 99.4775 88.0475) (end 99.06 87.63) (width 0.25) (layer F.Cu) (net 3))
 (segment (start 99.4775 92.075) (end 99.4775 88.0475) (width 0.25) (layer F.Cu) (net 3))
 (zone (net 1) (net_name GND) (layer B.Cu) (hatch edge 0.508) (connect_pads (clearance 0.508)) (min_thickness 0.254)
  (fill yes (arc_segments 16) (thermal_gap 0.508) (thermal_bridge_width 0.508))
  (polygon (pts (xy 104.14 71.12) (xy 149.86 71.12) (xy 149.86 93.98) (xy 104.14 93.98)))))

